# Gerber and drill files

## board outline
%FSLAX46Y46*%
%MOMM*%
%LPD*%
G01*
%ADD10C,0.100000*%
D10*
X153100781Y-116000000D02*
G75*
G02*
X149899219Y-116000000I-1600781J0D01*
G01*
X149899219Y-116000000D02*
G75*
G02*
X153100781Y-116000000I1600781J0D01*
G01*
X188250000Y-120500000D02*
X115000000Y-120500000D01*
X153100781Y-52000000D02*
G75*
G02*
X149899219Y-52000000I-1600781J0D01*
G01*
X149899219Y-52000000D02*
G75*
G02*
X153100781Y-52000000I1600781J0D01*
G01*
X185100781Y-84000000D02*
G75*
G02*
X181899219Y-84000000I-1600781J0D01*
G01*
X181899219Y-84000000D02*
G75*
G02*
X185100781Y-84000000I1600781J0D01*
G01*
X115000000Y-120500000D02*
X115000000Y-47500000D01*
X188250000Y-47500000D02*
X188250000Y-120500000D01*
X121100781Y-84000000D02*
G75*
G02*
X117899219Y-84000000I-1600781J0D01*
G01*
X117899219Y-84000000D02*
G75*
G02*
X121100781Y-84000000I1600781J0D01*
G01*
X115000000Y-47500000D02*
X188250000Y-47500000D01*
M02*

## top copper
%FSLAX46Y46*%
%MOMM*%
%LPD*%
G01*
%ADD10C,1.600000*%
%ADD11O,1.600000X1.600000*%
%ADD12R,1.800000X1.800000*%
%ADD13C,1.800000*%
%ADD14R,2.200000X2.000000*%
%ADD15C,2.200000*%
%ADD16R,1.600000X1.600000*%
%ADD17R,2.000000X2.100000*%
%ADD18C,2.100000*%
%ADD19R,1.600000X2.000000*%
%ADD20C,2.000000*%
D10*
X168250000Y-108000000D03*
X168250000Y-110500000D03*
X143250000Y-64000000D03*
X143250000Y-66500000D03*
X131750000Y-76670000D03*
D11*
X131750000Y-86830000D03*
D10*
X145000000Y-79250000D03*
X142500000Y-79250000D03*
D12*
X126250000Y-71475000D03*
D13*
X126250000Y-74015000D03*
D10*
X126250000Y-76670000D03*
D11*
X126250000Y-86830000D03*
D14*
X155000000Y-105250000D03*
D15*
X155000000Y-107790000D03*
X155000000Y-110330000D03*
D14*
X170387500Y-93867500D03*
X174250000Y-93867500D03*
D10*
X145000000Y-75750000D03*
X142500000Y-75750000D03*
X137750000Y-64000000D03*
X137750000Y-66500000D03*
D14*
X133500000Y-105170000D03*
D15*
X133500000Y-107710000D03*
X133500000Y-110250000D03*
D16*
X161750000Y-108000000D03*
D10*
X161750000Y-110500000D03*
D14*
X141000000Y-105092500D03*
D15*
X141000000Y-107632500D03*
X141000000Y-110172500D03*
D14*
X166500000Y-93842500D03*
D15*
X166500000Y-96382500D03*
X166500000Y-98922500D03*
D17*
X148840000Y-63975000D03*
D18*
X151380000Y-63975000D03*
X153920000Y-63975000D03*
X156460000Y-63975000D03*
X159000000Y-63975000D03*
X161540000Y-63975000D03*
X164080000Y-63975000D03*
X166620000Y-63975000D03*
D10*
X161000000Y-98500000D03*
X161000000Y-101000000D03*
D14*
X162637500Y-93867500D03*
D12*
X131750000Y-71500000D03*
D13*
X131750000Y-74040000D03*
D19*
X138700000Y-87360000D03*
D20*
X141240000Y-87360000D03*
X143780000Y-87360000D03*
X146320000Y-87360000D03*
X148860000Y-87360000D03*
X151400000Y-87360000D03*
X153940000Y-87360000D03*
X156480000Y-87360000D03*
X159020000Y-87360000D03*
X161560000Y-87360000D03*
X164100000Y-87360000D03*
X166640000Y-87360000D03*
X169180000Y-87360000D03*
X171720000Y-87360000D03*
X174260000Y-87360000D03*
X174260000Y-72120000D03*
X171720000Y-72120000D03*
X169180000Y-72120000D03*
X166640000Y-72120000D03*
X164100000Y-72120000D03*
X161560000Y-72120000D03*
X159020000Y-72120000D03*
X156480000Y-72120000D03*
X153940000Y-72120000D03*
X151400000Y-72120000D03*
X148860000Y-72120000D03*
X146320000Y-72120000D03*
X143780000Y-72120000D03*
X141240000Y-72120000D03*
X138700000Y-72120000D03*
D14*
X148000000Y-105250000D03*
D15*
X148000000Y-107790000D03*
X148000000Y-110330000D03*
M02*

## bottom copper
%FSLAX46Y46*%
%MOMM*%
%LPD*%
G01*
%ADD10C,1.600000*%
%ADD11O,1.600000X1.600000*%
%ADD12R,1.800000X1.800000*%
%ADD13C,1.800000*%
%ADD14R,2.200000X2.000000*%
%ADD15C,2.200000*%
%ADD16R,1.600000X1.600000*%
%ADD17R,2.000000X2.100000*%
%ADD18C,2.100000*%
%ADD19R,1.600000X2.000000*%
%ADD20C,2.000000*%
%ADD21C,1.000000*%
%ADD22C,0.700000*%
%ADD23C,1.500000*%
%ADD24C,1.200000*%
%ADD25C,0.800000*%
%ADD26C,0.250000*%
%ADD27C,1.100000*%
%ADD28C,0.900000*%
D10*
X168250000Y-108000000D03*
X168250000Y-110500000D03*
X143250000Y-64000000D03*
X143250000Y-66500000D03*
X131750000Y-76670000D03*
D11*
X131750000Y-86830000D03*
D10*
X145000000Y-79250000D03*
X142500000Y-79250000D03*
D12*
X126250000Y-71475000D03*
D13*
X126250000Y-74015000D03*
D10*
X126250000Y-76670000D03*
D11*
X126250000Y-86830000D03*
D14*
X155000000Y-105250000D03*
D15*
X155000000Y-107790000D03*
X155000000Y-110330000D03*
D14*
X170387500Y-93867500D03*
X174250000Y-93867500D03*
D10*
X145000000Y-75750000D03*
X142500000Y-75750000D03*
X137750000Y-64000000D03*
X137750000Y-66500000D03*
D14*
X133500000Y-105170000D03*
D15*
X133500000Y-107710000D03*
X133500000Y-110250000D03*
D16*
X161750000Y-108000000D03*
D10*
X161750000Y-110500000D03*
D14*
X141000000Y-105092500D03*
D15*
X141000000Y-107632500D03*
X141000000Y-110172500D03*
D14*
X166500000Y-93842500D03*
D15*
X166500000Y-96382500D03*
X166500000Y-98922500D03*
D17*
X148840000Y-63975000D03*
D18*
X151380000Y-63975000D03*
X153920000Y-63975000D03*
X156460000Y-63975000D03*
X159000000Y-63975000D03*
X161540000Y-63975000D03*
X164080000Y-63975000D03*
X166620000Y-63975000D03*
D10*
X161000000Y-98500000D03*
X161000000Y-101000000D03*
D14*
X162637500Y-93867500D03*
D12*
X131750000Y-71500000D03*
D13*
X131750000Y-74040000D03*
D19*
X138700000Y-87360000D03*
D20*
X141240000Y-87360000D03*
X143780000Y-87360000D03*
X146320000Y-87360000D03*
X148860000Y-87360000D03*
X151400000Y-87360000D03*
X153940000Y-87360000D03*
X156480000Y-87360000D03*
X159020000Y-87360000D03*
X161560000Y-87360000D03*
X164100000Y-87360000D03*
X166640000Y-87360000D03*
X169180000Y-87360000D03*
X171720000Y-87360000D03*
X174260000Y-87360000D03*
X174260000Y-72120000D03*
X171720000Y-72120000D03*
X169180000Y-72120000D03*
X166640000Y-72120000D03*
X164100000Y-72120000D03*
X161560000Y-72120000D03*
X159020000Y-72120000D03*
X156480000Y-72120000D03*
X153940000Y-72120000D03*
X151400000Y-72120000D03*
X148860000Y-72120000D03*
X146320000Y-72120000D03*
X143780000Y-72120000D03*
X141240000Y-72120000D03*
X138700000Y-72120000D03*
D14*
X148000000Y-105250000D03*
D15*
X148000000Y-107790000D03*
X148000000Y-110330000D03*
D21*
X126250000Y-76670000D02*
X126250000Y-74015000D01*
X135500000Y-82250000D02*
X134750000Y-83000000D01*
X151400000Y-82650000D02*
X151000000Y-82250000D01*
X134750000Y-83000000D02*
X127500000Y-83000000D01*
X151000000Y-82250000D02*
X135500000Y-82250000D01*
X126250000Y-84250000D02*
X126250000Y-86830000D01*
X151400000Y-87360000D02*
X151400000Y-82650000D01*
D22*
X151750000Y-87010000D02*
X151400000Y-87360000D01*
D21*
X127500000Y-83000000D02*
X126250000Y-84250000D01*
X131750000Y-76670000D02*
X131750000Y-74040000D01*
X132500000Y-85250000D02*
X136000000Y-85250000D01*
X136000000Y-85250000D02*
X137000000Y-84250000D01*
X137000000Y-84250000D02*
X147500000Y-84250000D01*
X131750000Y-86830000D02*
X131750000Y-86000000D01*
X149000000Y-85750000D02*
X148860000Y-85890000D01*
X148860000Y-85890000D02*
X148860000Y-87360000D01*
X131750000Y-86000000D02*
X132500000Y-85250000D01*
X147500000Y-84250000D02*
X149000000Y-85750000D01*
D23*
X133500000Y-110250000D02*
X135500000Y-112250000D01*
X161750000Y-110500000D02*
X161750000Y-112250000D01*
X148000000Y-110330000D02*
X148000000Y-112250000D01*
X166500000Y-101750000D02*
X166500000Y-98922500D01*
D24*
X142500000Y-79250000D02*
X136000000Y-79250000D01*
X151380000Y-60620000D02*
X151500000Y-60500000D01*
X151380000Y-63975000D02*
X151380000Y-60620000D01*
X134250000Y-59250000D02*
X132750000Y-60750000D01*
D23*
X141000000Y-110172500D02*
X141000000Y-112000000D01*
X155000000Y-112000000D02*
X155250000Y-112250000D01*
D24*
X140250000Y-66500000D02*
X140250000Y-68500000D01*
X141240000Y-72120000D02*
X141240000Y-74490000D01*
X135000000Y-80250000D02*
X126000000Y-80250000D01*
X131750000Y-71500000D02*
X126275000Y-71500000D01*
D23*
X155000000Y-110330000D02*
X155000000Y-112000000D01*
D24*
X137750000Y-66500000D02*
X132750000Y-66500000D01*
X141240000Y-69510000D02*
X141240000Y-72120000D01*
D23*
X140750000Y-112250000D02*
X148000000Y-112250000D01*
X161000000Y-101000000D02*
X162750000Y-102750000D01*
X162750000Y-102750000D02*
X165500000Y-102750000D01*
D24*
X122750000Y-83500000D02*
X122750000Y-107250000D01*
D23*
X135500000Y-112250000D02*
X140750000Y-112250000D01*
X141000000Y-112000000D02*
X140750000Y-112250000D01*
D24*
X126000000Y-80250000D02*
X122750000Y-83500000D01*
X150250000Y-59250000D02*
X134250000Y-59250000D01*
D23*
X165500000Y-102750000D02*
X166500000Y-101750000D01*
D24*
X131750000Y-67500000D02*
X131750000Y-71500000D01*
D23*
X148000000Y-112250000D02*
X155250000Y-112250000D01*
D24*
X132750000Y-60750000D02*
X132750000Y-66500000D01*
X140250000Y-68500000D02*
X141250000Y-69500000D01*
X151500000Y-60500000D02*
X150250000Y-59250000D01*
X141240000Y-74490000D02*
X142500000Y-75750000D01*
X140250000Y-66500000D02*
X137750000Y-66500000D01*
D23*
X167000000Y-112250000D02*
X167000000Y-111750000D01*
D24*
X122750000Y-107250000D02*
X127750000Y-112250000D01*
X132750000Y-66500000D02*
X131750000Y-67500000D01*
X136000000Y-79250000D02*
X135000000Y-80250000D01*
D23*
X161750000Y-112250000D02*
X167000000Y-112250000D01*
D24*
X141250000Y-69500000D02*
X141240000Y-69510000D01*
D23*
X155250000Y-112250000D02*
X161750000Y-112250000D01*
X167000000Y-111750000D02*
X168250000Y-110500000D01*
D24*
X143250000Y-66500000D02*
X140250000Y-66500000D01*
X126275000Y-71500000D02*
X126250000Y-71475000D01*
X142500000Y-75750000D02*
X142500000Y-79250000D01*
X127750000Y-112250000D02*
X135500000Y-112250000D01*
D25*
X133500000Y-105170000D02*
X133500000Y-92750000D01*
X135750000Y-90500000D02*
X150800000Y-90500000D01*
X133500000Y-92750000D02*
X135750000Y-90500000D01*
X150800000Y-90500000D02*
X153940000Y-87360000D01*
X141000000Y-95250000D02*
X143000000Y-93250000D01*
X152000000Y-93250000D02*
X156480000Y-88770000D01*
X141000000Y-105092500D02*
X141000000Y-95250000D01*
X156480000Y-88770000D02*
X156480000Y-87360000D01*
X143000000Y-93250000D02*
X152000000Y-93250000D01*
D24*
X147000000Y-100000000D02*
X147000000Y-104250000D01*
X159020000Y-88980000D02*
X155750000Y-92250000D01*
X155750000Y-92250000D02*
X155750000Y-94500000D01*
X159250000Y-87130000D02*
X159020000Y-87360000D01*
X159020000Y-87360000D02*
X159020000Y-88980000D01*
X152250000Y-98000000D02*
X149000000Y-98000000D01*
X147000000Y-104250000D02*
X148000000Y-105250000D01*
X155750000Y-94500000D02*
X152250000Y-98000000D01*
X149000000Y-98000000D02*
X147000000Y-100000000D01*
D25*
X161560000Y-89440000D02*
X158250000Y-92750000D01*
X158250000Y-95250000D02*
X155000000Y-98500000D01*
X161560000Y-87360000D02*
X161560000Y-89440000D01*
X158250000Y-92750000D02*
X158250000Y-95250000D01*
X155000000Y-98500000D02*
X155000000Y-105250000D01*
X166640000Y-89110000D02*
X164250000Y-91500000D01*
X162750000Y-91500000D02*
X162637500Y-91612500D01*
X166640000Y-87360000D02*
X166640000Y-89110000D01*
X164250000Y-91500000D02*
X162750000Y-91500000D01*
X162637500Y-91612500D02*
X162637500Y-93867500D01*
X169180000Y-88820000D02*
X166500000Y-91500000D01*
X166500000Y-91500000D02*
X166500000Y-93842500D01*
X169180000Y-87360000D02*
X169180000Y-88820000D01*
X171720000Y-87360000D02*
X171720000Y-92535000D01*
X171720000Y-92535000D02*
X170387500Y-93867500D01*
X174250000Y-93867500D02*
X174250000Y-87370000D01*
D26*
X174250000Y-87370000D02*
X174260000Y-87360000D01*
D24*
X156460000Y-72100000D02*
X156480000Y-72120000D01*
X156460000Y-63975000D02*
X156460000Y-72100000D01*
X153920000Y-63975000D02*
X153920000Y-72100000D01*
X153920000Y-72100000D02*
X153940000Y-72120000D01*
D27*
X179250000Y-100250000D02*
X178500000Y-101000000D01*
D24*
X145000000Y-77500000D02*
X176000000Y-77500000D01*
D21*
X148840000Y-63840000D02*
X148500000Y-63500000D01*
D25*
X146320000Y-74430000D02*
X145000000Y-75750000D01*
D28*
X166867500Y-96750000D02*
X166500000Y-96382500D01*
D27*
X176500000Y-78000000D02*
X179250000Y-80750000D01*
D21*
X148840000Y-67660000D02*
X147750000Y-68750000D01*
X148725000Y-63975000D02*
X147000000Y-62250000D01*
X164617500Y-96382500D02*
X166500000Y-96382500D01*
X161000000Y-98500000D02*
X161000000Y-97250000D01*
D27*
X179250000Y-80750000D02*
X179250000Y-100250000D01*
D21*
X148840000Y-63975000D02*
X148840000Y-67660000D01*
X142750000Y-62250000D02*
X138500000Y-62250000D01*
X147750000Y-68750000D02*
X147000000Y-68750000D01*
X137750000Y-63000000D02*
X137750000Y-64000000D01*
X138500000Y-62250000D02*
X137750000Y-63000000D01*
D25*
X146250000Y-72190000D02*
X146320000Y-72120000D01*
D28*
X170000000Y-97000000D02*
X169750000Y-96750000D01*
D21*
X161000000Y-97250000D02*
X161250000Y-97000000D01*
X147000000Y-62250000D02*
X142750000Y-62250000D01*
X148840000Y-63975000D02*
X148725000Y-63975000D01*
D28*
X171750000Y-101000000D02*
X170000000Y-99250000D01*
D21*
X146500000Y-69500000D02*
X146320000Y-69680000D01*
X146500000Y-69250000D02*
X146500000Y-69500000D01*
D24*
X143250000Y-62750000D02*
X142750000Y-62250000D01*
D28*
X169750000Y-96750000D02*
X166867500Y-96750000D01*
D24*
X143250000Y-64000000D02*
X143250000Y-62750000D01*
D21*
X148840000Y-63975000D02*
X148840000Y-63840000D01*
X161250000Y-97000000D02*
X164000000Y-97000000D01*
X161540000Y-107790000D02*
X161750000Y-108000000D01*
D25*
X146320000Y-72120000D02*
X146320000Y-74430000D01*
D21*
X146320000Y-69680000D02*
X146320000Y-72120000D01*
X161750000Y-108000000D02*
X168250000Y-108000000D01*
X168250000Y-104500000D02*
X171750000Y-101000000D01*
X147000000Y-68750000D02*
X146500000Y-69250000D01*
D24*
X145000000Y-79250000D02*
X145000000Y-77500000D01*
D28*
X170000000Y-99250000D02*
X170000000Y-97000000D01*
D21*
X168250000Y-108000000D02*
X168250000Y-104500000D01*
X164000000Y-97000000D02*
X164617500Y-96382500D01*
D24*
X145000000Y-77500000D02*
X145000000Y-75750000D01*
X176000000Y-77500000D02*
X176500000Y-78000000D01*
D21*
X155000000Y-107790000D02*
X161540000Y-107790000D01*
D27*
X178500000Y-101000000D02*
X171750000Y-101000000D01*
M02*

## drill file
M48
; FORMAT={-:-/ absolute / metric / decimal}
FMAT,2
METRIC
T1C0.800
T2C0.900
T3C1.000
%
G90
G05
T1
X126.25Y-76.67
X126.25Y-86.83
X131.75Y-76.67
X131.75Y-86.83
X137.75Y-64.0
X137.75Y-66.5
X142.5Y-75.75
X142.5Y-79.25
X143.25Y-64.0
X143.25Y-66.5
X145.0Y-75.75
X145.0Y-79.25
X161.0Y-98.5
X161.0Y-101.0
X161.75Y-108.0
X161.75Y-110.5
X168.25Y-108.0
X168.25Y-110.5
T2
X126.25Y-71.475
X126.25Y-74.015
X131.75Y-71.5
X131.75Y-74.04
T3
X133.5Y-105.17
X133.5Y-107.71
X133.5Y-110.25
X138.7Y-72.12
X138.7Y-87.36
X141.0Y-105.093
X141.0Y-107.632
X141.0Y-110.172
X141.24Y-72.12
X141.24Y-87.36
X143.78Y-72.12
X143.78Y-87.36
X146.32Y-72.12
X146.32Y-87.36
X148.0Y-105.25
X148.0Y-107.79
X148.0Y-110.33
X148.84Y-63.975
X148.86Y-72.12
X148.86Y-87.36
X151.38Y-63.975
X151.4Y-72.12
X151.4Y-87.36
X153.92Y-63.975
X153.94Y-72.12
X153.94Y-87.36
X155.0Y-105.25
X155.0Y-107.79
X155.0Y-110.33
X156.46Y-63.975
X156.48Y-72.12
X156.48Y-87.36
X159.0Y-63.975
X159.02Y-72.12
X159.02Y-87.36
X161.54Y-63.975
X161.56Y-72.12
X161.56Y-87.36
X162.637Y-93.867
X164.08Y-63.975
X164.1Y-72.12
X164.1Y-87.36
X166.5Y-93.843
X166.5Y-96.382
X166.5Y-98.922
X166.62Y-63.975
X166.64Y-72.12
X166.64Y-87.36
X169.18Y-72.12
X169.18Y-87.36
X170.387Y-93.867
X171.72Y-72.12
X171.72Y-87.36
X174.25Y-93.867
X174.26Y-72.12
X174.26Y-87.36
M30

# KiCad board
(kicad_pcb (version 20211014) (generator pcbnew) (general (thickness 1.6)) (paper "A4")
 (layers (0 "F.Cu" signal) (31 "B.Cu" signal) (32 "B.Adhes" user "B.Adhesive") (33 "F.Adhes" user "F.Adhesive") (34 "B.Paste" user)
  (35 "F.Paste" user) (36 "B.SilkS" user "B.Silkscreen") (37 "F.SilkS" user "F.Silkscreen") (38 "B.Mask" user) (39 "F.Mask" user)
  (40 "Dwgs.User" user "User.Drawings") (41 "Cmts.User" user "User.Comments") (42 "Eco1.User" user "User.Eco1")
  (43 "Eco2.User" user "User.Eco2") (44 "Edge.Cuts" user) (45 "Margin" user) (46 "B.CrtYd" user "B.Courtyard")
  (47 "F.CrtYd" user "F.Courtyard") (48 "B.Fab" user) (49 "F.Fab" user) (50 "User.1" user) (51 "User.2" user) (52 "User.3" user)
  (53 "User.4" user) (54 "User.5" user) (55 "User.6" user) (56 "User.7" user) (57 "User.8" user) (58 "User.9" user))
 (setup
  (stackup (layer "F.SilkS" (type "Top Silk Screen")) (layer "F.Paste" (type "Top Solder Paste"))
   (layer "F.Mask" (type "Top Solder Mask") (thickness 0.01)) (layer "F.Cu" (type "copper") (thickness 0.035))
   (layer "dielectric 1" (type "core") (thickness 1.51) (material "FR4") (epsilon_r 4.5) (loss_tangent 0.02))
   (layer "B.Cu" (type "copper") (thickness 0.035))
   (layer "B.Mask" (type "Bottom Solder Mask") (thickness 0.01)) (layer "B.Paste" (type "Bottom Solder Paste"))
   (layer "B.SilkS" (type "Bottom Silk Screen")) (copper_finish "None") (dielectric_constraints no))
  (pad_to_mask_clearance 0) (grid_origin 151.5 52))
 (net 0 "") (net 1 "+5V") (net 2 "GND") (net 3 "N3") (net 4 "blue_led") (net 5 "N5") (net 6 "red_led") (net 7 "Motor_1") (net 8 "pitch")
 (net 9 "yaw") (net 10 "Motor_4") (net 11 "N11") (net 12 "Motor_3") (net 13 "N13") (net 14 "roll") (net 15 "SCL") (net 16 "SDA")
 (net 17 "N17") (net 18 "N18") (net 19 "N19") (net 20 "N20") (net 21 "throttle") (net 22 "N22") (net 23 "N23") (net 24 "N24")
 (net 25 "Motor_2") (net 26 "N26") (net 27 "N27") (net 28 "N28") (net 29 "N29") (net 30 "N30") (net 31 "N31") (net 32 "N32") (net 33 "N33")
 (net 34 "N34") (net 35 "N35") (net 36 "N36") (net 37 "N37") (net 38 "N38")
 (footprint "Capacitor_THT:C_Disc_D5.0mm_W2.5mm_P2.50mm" (layer "F.Cu") (at 168.25 108 -90)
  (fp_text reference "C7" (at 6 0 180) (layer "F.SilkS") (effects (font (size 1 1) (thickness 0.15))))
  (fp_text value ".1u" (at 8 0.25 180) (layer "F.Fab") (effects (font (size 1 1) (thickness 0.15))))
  (pad "1" thru_hole circle (at 0 0 270) (size 1.6 1.6) (drill 0.8) (layers *.Cu *.Mask) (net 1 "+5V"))
  (pad "2" thru_hole circle (at 2.5 0 270) (size 1.6 1.6) (drill 0.8) (layers *.Cu *.Mask) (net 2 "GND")))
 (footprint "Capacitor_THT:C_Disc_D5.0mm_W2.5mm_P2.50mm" (layer "F.Cu") (at 143.25 64 -90)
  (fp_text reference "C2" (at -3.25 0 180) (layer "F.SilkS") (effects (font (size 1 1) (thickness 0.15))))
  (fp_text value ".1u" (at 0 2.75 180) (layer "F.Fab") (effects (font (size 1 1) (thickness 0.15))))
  (pad "1" thru_hole circle (at 0 0 270) (size 1.6 1.6) (drill 0.8) (layers *.Cu *.Mask) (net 1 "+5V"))
  (pad "2" thru_hole circle (at 2.5 0 270) (size 1.6 1.6) (drill 0.8) (layers *.Cu *.Mask) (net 2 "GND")))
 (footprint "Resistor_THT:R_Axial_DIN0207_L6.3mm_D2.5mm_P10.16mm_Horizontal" (layer "F.Cu") (at 131.75 76.67 -90)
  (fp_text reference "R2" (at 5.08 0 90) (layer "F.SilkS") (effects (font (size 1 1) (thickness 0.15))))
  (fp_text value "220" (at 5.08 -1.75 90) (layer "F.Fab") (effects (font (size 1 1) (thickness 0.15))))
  (pad "1" thru_hole circle (at 0 0 270) (size 1.6 1.6) (drill 0.8) (layers *.Cu *.Mask) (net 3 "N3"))
  (pad "2" thru_hole oval (at 10.16 0 270) (size 1.6 1.6) (drill 0.8) (layers *.Cu *.Mask) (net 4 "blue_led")))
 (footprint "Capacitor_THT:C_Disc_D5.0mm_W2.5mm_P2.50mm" (layer "F.Cu") (at 145 79.25 180)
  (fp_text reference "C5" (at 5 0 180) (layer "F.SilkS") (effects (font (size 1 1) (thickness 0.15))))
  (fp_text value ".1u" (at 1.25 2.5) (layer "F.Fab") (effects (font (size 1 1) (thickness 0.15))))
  (pad "1" thru_hole circle (at 0 0 180) (size 1.6 1.6) (drill 0.8) (layers *.Cu *.Mask) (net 1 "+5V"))
  (pad "2" thru_hole circle (at 2.5 0 180) (size 1.6 1.6) (drill 0.8) (layers *.Cu *.Mask) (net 2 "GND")))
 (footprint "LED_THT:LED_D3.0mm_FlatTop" (layer "F.Cu") (at 126.25 71.475 -90)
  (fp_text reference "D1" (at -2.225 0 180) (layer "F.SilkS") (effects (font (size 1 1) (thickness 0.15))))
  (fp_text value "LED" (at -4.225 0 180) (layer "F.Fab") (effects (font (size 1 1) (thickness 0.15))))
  (pad "1" thru_hole rect (at 0 0 270) (size 1.8 1.8) (drill 0.9) (layers *.Cu *.Mask) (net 2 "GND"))
  (pad "2" thru_hole circle (at 2.54 0 270) (size 1.8 1.8) (drill 0.9) (layers *.Cu *.Mask) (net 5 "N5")))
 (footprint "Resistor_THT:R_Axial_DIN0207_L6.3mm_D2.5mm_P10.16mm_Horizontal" (layer "F.Cu") (at 126.25 76.67 -90)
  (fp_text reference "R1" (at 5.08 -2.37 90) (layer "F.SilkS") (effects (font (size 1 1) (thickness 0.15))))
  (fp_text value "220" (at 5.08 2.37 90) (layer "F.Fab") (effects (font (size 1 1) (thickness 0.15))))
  (pad "1" thru_hole circle (at 0 0 270) (size 1.6 1.6) (drill 0.8) (layers *.Cu *.Mask) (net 5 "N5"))
  (pad "2" thru_hole oval (at 10.16 0 270) (size 1.6 1.6) (drill 0.8) (layers *.Cu *.Mask) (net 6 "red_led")))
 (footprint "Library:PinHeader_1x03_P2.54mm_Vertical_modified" (layer "F.Cu") (at 156.33 114.14)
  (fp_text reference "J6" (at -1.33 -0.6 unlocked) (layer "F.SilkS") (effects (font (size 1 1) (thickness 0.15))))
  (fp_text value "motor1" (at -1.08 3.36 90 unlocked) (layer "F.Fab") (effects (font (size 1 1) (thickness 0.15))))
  (pad "1" thru_hole rect (at -1.33 -8.89) (size 2.2 2) (drill 1) (layers *.Cu *.Mask) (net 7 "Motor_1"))
  (pad "2" thru_hole circle (at -1.33 -6.35) (size 2.2 2.2) (drill 1) (layers *.Cu *.Mask) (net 1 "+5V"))
  (pad "3" thru_hole circle (at -1.33 -3.81) (size 2.2 2.2) (drill 1) (layers *.Cu *.Mask) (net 2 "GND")))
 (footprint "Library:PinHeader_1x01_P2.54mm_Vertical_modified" (layer "F.Cu") (at 172.1875 98.2075)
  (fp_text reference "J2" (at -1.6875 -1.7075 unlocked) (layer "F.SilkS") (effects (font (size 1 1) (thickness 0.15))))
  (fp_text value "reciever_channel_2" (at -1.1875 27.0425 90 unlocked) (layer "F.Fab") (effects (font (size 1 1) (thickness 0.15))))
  (pad "1" thru_hole rect (at -1.8 -4.34) (size 2.2 2) (drill 1) (layers *.Cu *.Mask) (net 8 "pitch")))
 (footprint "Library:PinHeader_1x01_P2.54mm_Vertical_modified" (layer "F.Cu") (at 176.05 98.2075)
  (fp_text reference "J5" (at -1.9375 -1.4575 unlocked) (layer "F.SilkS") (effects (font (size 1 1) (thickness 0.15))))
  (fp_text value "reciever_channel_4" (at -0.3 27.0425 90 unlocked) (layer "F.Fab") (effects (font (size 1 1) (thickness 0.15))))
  (pad "1" thru_hole rect (at -1.8 -4.34) (size 2.2 2) (drill 1) (layers *.Cu *.Mask) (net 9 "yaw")))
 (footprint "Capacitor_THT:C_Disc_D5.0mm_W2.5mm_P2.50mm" (layer "F.Cu") (at 145 75.75 180)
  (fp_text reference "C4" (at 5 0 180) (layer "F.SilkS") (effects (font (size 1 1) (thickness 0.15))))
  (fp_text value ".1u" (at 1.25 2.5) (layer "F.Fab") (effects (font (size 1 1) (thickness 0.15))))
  (pad "1" thru_hole circle (at 0 0 180) (size 1.6 1.6) (drill 0.8) (layers *.Cu *.Mask) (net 1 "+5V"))
  (pad "2" thru_hole circle (at 2.5 0 180) (size 1.6 1.6) (drill 0.8) (layers *.Cu *.Mask) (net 2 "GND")))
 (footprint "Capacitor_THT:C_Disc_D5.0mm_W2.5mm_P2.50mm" (layer "F.Cu") (at 137.75 64 -90)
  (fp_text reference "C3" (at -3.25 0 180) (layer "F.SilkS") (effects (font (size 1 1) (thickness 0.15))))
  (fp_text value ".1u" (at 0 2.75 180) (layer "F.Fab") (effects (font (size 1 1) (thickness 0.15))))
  (pad "1" thru_hole circle (at 0 0 270) (size 1.6 1.6) (drill 0.8) (layers *.Cu *.Mask) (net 1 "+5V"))
  (pad "2" thru_hole circle (at 2.5 0 270) (size 1.6 1.6) (drill 0.8) (layers *.Cu *.Mask) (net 2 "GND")))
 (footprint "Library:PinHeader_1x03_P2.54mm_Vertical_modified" (layer "F.Cu") (at 134.83 114.06)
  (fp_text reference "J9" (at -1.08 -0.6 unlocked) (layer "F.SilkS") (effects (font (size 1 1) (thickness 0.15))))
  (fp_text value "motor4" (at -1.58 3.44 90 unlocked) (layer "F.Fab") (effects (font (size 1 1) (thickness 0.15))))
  (pad "1" thru_hole rect (at -1.33 -8.89) (size 2.2 2) (drill 1) (layers *.Cu *.Mask) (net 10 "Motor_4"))
  (pad "2" thru_hole circle (at -1.33 -6.35) (size 2.2 2.2) (drill 1) (layers *.Cu *.Mask) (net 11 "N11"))
  (pad "3" thru_hole circle (at -1.33 -3.81) (size 2.2 2.2) (drill 1) (layers *.Cu *.Mask) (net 2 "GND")))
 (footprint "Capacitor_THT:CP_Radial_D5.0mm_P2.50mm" (layer "F.Cu") (at 161.75 108 -90)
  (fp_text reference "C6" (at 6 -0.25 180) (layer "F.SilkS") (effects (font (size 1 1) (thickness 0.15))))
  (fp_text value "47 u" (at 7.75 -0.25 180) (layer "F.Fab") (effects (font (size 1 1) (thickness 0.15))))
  (pad "1" thru_hole rect (at 0 0 270) (size 1.6 1.6) (drill 0.8) (layers *.Cu *.Mask) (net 1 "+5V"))
  (pad "2" thru_hole circle (at 2.5 0 270) (size 1.6 1.6) (drill 0.8) (layers *.Cu *.Mask) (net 2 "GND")))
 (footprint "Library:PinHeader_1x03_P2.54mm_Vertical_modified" (layer "F.Cu") (at 142.33 113.9825)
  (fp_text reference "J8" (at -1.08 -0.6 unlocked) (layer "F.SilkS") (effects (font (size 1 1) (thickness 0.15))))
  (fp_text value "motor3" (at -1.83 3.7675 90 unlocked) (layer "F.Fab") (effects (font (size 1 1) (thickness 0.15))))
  (pad "1" thru_hole rect (at -1.33 -8.89) (size 2.2 2) (drill 1) (layers *.Cu *.Mask) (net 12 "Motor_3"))
  (pad "2" thru_hole circle (at -1.33 -6.35) (size 2.2 2.2) (drill 1) (layers *.Cu *.Mask) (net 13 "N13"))
  (pad "3" thru_hole circle (at -1.33 -3.81) (size 2.2 2.2) (drill 1) (layers *.Cu *.Mask) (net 2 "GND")))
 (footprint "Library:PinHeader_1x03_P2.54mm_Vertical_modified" (layer "F.Cu") (at 167.83 102.7325)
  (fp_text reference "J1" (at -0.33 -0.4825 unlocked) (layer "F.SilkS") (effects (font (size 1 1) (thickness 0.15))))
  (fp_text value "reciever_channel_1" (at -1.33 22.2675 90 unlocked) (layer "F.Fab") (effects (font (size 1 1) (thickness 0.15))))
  (pad "1" thru_hole rect (at -1.33 -8.89) (size 2.2 2) (drill 1) (layers *.Cu *.Mask) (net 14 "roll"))
  (pad "2" thru_hole circle (at -1.33 -6.35) (size 2.2 2.2) (drill 1) (layers *.Cu *.Mask) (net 1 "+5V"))
  (pad "3" thru_hole circle (at -1.33 -3.81) (size 2.2 2.2) (drill 1) (layers *.Cu *.Mask) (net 2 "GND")))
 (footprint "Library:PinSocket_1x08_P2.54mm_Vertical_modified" (layer "F.Cu") (at 170.49 65.185 90)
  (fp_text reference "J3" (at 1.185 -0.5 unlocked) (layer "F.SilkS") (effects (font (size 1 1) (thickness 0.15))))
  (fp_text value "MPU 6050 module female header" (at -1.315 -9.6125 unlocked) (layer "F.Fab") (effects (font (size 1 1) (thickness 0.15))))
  (pad "1" thru_hole rect (at 1.21 -21.65 90) (size 2.1 2) (drill 1) (layers *.Cu *.Mask) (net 1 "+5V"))
  (pad "2" thru_hole circle (at 1.21 -19.11 90) (size 2.1 2.1) (drill 1) (layers *.Cu *.Mask) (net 2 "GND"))
  (pad "3" thru_hole circle (at 1.21 -16.57 90) (size 2.1 2.1) (drill 1) (layers *.Cu *.Mask) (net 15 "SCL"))
  (pad "4" thru_hole circle (at 1.21 -14.03 90) (size 2.1 2.1) (drill 1) (layers *.Cu *.Mask) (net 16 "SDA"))
  (pad "5" thru_hole circle (at 1.21 -11.49 90) (size 2.1 2.1) (drill 1) (layers *.Cu *.Mask) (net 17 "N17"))
  (pad "6" thru_hole circle (at 1.21 -8.95 90) (size 2.1 2.1) (drill 1) (layers *.Cu *.Mask) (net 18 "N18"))
  (pad "7" thru_hole circle (at 1.21 -6.41 90) (size 2.1 2.1) (drill 1) (layers *.Cu *.Mask) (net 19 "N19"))
  (pad "8" thru_hole circle (at 1.21 -3.87 90) (size 2.1 2.1) (drill 1) (layers *.Cu *.Mask) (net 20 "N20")))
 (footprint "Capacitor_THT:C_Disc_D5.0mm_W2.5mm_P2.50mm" (layer "F.Cu") (at 161 98.5 -90)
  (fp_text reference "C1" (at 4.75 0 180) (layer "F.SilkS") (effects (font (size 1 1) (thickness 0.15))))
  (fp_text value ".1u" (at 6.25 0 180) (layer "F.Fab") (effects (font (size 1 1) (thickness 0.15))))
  (pad "1" thru_hole circle (at 0 0 270) (size 1.6 1.6) (drill 0.8) (layers *.Cu *.Mask) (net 1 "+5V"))
  (pad "2" thru_hole circle (at 2.5 0 270) (size 1.6 1.6) (drill 0.8) (layers *.Cu *.Mask) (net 2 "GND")))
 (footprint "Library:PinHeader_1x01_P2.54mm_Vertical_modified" (layer "F.Cu") (at 164.4375 98.2075)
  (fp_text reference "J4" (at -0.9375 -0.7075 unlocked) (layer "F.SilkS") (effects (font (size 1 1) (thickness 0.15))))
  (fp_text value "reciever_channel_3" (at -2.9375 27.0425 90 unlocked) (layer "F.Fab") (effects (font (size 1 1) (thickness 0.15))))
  (pad "1" thru_hole rect (at -1.8 -4.34) (size 2.2 2) (drill 1) (layers *.Cu *.Mask) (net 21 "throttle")))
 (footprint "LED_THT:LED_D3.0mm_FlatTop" (layer "F.Cu") (at 131.75 71.5 -90)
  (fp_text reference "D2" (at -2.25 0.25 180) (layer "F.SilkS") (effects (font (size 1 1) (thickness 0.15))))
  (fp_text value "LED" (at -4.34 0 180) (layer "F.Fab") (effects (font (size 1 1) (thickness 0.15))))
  (pad "1" thru_hole rect (at 0 0 270) (size 1.8 1.8) (drill 0.9) (layers *.Cu *.Mask) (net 2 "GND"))
  (pad "2" thru_hole circle (at 2.54 0 270) (size 1.8 1.8) (drill 0.9) (layers *.Cu *.Mask) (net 3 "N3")))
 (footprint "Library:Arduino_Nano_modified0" (layer "F.Cu") (at 138.7 87.36 90)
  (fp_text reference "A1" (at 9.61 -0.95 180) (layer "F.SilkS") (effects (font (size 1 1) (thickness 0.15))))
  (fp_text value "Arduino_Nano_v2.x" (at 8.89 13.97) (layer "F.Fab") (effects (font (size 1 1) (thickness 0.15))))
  (pad "1" thru_hole rect (at 0 0 90) (size 2 1.6) (drill 1) (layers *.Cu *.Mask) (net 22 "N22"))
  (pad "2" thru_hole circle (at 0 2.54 90) (size 2 2) (drill 1) (layers *.Cu *.Mask) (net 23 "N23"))
  (pad "3" thru_hole circle (at 0 5.08 90) (size 2 2) (drill 1) (layers *.Cu *.Mask) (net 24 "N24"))
  (pad "4" thru_hole circle (at 0 7.62 90) (size 2 2) (drill 1) (layers *.Cu *.Mask) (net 2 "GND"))
  (pad "5" thru_hole circle (at 0 10.16 90) (size 2 2) (drill 1) (layers *.Cu *.Mask) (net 4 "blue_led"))
  (pad "6" thru_hole circle (at 0 12.7 90) (size 2 2) (drill 1) (layers *.Cu *.Mask) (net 6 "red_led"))
  (pad "7" thru_hole circle (at 0 15.24 90) (size 2 2) (drill 1) (layers *.Cu *.Mask) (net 10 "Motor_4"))
  (pad "8" thru_hole circle (at 0 17.78 90) (size 2 2) (drill 1) (layers *.Cu *.Mask) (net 12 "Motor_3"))
  (pad "9" thru_hole circle (at 0 20.32 90) (size 2 2) (drill 1) (layers *.Cu *.Mask) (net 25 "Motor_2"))
  (pad "10" thru_hole circle (at 0 22.86 90) (size 2 2) (drill 1) (layers *.Cu *.Mask) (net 7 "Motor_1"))
  (pad "11" thru_hole circle (at 0 25.4 90) (size 2 2) (drill 1) (layers *.Cu *.Mask) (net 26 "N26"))
  (pad "12" thru_hole circle (at 0 27.94 90) (size 2 2) (drill 1) (layers *.Cu *.Mask) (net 21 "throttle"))
  (pad "13" thru_hole circle (at 0 30.48 90) (size 2 2) (drill 1) (layers *.Cu *.Mask) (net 14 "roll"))
  (pad "14" thru_hole circle (at 0 33.02 90) (size 2 2) (drill 1) (layers *.Cu *.Mask) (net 8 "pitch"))
  (pad "15" thru_hole circle (at 0 35.56 90) (size 2 2) (drill 1) (layers *.Cu *.Mask) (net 9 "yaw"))
  (pad "16" thru_hole circle (at 15.24 35.56 90) (size 2 2) (drill 1) (layers *.Cu *.Mask) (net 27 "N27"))
  (pad "17" thru_hole circle (at 15.24 33.02 90) (size 2 2) (drill 1) (layers *.Cu *.Mask) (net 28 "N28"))
  (pad "18" thru_hole circle (at 15.24 30.48 90) (size 2 2) (drill 1) (layers *.Cu *.Mask) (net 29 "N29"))
  (pad "19" thru_hole circle (at 15.24 27.94 90) (size 2 2) (drill 1) (layers *.Cu *.Mask) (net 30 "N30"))
  (pad "20" thru_hole circle (at 15.24 25.4 90) (size 2 2) (drill 1) (layers *.Cu *.Mask) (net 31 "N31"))
  (pad "21" thru_hole circle (at 15.24 22.86 90) (size 2 2) (drill 1) (layers *.Cu *.Mask) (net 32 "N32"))
  (pad "22" thru_hole circle (at 15.24 20.32 90) (size 2 2) (drill 1) (layers *.Cu *.Mask) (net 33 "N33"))
  (pad "23" thru_hole circle (at 15.24 17.78 90) (size 2 2) (drill 1) (layers *.Cu *.Mask) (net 16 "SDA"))
  (pad "24" thru_hole circle (at 15.24 15.24 90) (size 2 2) (drill 1) (layers *.Cu *.Mask) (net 15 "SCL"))
  (pad "25" thru_hole circle (at 15.24 12.7 90) (size 2 2) (drill 1) (layers *.Cu *.Mask) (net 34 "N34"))
  (pad "26" thru_hole circle (at 15.24 10.16 90) (size 2 2) (drill 1) (layers *.Cu *.Mask) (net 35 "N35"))
  (pad "27" thru_hole circle (at 15.24 7.62 90) (size 2 2) (drill 1) (layers *.Cu *.Mask) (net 1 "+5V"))
  (pad "28" thru_hole circle (at 15.24 5.08 90) (size 2 2) (drill 1) (layers *.Cu *.Mask) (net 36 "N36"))
  (pad "29" thru_hole circle (at 15.24 2.54 90) (size 2 2) (drill 1) (layers *.Cu *.Mask) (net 2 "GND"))
  (pad "30" thru_hole circle (at 15.24 0 90) (size 2 2) (drill 1) (layers *.Cu *.Mask) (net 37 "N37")))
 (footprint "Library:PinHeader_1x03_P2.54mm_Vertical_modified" (layer "F.Cu") (at 149.33 114.14)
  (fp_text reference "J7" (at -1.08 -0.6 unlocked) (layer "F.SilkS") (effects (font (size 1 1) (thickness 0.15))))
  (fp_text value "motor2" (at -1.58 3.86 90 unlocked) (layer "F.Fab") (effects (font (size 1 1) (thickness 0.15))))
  (pad "1" thru_hole rect (at -1.33 -8.89) (size 2.2 2) (drill 1) (layers *.Cu *.Mask) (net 25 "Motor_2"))
  (pad "2" thru_hole circle (at -1.33 -6.35) (size 2.2 2.2) (drill 1) (layers *.Cu *.Mask) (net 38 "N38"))
  (pad "3" thru_hole circle (at -1.33 -3.81) (size 2.2 2.2) (drill 1) (layers *.Cu *.Mask) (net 2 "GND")))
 (gr_circle (center 151.5 116) (end 152.75 115) (layer "Edge.Cuts") (width 0.1) (fill none))
 (gr_line (start 188.25 120.5) (end 115 120.5) (layer "Edge.Cuts") (width 0.1))
 (gr_circle (center 151.5 52) (end 152.75 51) (layer "Edge.Cuts") (width 0.1) (fill none))
 (gr_circle (center 183.5 84) (end 184.5 82.75) (layer "Edge.Cuts") (width 0.1) (fill none))
 (gr_line (start 115 120.5) (end 115 47.5) (layer "Edge.Cuts") (width 0.1))
 (gr_line (start 188.25 47.5) (end 188.25 120.5) (layer "Edge.Cuts") (width 0.1))
 (gr_circle (center 119.5 84) (end 120.5 82.75) (layer "Edge.Cuts") (width 0.1) (fill none))
 (gr_line (start 115 47.5) (end 188.25 47.5) (layer "Edge.Cuts") (width 0.1))
 (segment (start 126.25 76.67) (end 126.25 74.015) (width 1) (layer "B.Cu") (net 5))
 (segment (start 135.5 82.25) (end 134.75 83) (width 1) (layer "B.Cu") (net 6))
 (segment (start 151.4 82.65) (end 151 82.25) (width 1) (layer "B.Cu") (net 6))
 (segment (start 134.75 83) (end 127.5 83) (width 1) (layer "B.Cu") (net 6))
 (segment (start 151 82.25) (end 135.5 82.25) (width 1) (layer "B.Cu") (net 6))
 (segment (start 126.25 84.25) (end 126.25 86.83) (width 1) (layer "B.Cu") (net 6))
 (segment (start 151.4 87.36) (end 151.4 82.65) (width 1) (layer "B.Cu") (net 6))
 (segment (start 151.75 87.01) (end 151.4 87.36) (width 0.7) (layer "B.Cu") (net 6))
 (segment (start 127.5 83) (end 126.25 84.25) (width 1) (layer "B.Cu") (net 6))
 (segment (start 131.75 76.67) (end 131.75 74.04) (width 1) (layer "B.Cu") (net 3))
 (segment (start 132.5 85.25) (end 136 85.25) (width 1) (layer "B.Cu") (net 4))
 (segment (start 136 85.25) (end 137 84.25) (width 1) (layer "B.Cu") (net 4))
 (segment (start 137 84.25) (end 147.5 84.25) (width 1) (layer "B.Cu") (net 4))
 (segment (start 131.75 86.83) (end 131.75 86) (width 1) (layer "B.Cu") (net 4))
 (segment (start 149 85.75) (end 148.86 85.89) (width 1) (layer "B.Cu") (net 4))
 (segment (start 148.86 85.89) (end 148.86 87.36) (width 1) (layer "B.Cu") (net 4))
 (segment (start 131.75 86) (end 132.5 85.25) (width 1) (layer "B.Cu") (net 4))
 (segment (start 147.5 84.25) (end 149 85.75) (width 1) (layer "B.Cu") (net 4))
 (segment (start 133.5 110.25) (end 135.5 112.25) (width 1.5) (layer "B.Cu") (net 2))
 (segment (start 161.75 110.5) (end 161.75 112.25) (width 1.5) (layer "B.Cu") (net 2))
 (segment (start 148 110.33) (end 148 112.25) (width 1.5) (layer "B.Cu") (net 2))
 (segment (start 166.5 101.75) (end 166.5 98.9225) (width 1.5) (layer "B.Cu") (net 2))
 (segment (start 142.5 79.25) (end 136 79.25) (width 1.2) (layer "B.Cu") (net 2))
 (segment (start 151.38 60.62) (end 151.5 60.5) (width 1.2) (layer "B.Cu") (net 2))
 (segment (start 151.38 63.975) (end 151.38 60.62) (width 1.2) (layer "B.Cu") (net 2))
 (segment (start 134.25 59.25) (end 132.75 60.75) (width 1.2) (layer "B.Cu") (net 2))
 (segment (start 141 110.1725) (end 141 112) (width 1.5) (layer "B.Cu") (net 2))
 (segment (start 155 112) (end 155.25 112.25) (width 1.5) (layer "B.Cu") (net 2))
 (segment (start 140.25 66.5) (end 140.25 68.5) (width 1.2) (layer "B.Cu") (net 2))
 (segment (start 141.24 72.12) (end 141.24 74.49) (width 1.2) (layer "B.Cu") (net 2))
 (segment (start 135 80.25) (end 126 80.25) (width 1.2) (layer "B.Cu") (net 2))
 (segment (start 131.75 71.5) (end 126.275 71.5) (width 1.2) (layer "B.Cu") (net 2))
 (segment (start 155 110.33) (end 155 112) (width 1.5) (layer "B.Cu") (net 2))
 (segment (start 137.75 66.5) (end 132.75 66.5) (width 1.2) (layer "B.Cu") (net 2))
 (segment (start 141.24 69.51) (end 141.24 72.12) (width 1.2) (layer "B.Cu") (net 2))
 (segment (start 140.75 112.25) (end 148 112.25) (width 1.5) (layer "B.Cu") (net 2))
 (segment (start 161 101) (end 162.75 102.75) (width 1.5) (layer "B.Cu") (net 2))
 (segment (start 162.75 102.75) (end 165.5 102.75) (width 1.5) (layer "B.Cu") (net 2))
 (segment (start 122.75 83.5) (end 122.75 107.25) (width 1.2) (layer "B.Cu") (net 2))
 (segment (start 135.5 112.25) (end 140.75 112.25) (width 1.5) (layer "B.Cu") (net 2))
 (segment (start 141 112) (end 140.75 112.25) (width 1.5) (layer "B.Cu") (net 2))
 (segment (start 126 80.25) (end 122.75 83.5) (width 1.2) (layer "B.Cu") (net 2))
 (segment (start 150.25 59.25) (end 134.25 59.25) (width 1.2) (layer "B.Cu") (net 2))
 (segment (start 165.5 102.75) (end 166.5 101.75) (width 1.5) (layer "B.Cu") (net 2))
 (segment (start 131.75 67.5) (end 131.75 71.5) (width 1.2) (layer "B.Cu") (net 2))
 (segment (start 148 112.25) (end 155.25 112.25) (width 1.5) (layer "B.Cu") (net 2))
 (segment (start 132.75 60.75) (end 132.75 66.5) (width 1.2) (layer "B.Cu") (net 2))
 (segment (start 140.25 68.5) (end 141.25 69.5) (width 1.2) (layer "B.Cu") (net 2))
 (segment (start 151.5 60.5) (end 150.25 59.25) (width 1.2) (layer "B.Cu") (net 2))
 (segment (start 141.24 74.49) (end 142.5 75.75) (width 1.2) (layer "B.Cu") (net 2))
 (segment (start 140.25 66.5) (end 137.75 66.5) (width 1.2) (layer "B.Cu") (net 2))
 (segment (start 167 112.25) (end 167 111.75) (width 1.5) (layer "B.Cu") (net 2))
 (segment (start 122.75 107.25) (end 127.75 112.25) (width 1.2) (layer "B.Cu") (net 2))
 (segment (start 132.75 66.5) (end 131.75 67.5) (width 1.2) (layer "B.Cu") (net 2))
 (segment (start 136 79.25) (end 135 80.25) (width 1.2) (layer "B.Cu") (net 2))
 (segment (start 161.75 112.25) (end 167 112.25) (width 1.5) (layer "B.Cu") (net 2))
 (segment (start 141.25 69.5) (end 141.24 69.51) (width 1.2) (layer "B.Cu") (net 2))
 (segment (start 155.25 112.25) (end 161.75 112.25) (width 1.5) (layer "B.Cu") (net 2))
 (segment (start 167 111.75) (end 168.25 110.5) (width 1.5) (layer "B.Cu") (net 2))
 (segment (start 143.25 66.5) (end 140.25 66.5) (width 1.2) (layer "B.Cu") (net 2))
 (segment (start 126.275 71.5) (end 126.25 71.475) (width 1.2) (layer "B.Cu") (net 2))
 (segment (start 142.5 75.75) (end 142.5 79.25) (width 1.2) (layer "B.Cu") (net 2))
 (segment (start 127.75 112.25) (end 135.5 112.25) (width 1.2) (layer "B.Cu") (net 2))
 (segment (start 133.5 105.17) (end 133.5 92.75) (width 0.8) (layer "B.Cu") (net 10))
 (segment (start 135.75 90.5) (end 150.8 90.5) (width 0.8) (layer "B.Cu") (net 10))
 (segment (start 133.5 92.75) (end 135.75 90.5) (width 0.8) (layer "B.Cu") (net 10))
 (segment (start 150.8 90.5) (end 153.94 87.36) (width 0.8) (layer "B.Cu") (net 10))
 (segment (start 141 95.25) (end 143 93.25) (width 0.8) (layer "B.Cu") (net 12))
 (segment (start 152 93.25) (end 156.48 88.77) (width 0.8) (layer "B.Cu") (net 12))
 (segment (start 141 105.0925) (end 141 95.25) (width 0.8) (layer "B.Cu") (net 12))
 (segment (start 156.48 88.77) (end 156.48 87.36) (width 0.8) (layer "B.Cu") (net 12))
 (segment (start 143 93.25) (end 152 93.25) (width 0.8) (layer "B.Cu") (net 12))
 (segment (start 147 100) (end 147 104.25) (width 1.2) (layer "B.Cu") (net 25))
 (segment (start 159.02 88.98) (end 155.75 92.25) (width 1.2) (layer "B.Cu") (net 25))
 (segment (start 155.75 92.25) (end 155.75 94.5) (width 1.2) (layer "B.Cu") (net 25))
 (segment (start 159.25 87.13) (end 159.02 87.36) (width 1.2) (layer "B.Cu") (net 25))
 (segment (start 159.02 87.36) (end 159.02 88.98) (width 1.2) (layer "B.Cu") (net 25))
 (segment (start 152.25 98) (end 149 98) (width 1.2) (layer "B.Cu") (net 25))
 (segment (start 147 104.25) (end 148 105.25) (width 1.2) (layer "B.Cu") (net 25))
 (segment (start 155.75 94.5) (end 152.25 98) (width 1.2) (layer "B.Cu") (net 25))
 (segment (start 149 98) (end 147 100) (width 1.2) (layer "B.Cu") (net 25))
 (segment (start 161.56 89.44) (end 158.25 92.75) (width 0.8) (layer "B.Cu") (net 7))
 (segment (start 158.25 95.25) (end 155 98.5) (width 0.8) (layer "B.Cu") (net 7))
 (segment (start 161.56 87.36) (end 161.56 89.44) (width 0.8) (layer "B.Cu") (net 7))
 (segment (start 158.25 92.75) (end 158.25 95.25) (width 0.8) (layer "B.Cu") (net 7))
 (segment (start 155 98.5) (end 155 105.25) (width 0.8) (layer "B.Cu") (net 7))
 (segment (start 166.64 89.11) (end 164.25 91.5) (width 0.8) (layer "B.Cu") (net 21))
 (segment (start 162.75 91.5) (end 162.6375 91.6125) (width 0.8) (layer "B.Cu") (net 21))
 (segment (start 166.64 87.36) (end 166.64 89.11) (width 0.8) (layer "B.Cu") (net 21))
 (segment (start 164.25 91.5) (end 162.75 91.5) (width 0.8) (layer "B.Cu") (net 21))
 (segment (start 162.6375 91.6125) (end 162.6375 93.8675) (width 0.8) (layer "B.Cu") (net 21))
 (segment (start 169.18 88.82) (end 166.5 91.5) (width 0.8) (layer "B.Cu") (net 14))
 (segment (start 166.5 91.5) (end 166.5 93.8425) (width 0.8) (layer "B.Cu") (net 14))
 (segment (start 169.18 87.36) (end 169.18 88.82) (width 0.8) (layer "B.Cu") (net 14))
 (segment (start 171.72 87.36) (end 171.72 92.535) (width 0.8) (layer "B.Cu") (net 8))
 (segment (start 171.72 92.535) (end 170.3875 93.8675) (width 0.8) (layer "B.Cu") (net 8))
 (segment (start 174.25 93.8675) (end 174.25 87.37) (width 0.8) (layer "B.Cu") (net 9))
 (segment (start 174.25 87.37) (end 174.26 87.36) (width 0.25) (layer "B.Cu") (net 9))
 (segment (start 156.46 72.1) (end 156.48 72.12) (width 1.2) (layer "B.Cu") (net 16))
 (segment (start 156.46 63.975) (end 156.46 72.1) (width 1.2) (layer "B.Cu") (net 16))
 (segment (start 153.92 63.975) (end 153.92 72.1) (width 1.2) (layer "B.Cu") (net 15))
 (segment (start 153.92 72.1) (end 153.94 72.12) (width 1.2) (layer "B.Cu") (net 15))
 (segment (start 179.25 100.25) (end 178.5 101) (width 1.1) (layer "B.Cu") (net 1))
 (segment (start 145 77.5) (end 176 77.5) (width 1.2) (layer "B.Cu") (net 1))
 (segment (start 148.84 63.84) (end 148.5 63.5) (width 1) (layer "B.Cu") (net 1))
 (segment (start 146.32 74.43) (end 145 75.75) (width 0.8) (layer "B.Cu") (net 1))
 (segment (start 166.8675 96.75) (end 166.5 96.3825) (width 0.9) (layer "B.Cu") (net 1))
 (segment (start 176.5 78) (end 179.25 80.75) (width 1.1) (layer "B.Cu") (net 1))
 (segment (start 148.84 67.66) (end 147.75 68.75) (width 1) (layer "B.Cu") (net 1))
 (segment (start 148.725 63.975) (end 147 62.25) (width 1) (layer "B.Cu") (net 1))
 (segment (start 164.6175 96.3825) (end 166.5 96.3825) (width 1) (layer "B.Cu") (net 1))
 (segment (start 161 98.5) (end 161 97.25) (width 1) (layer "B.Cu") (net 1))
 (segment (start 179.25 80.75) (end 179.25 100.25) (width 1.1) (layer "B.Cu") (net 1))
 (segment (start 148.84 63.975) (end 148.84 67.66) (width 1) (layer "B.Cu") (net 1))
 (segment (start 142.75 62.25) (end 138.5 62.25) (width 1) (layer "B.Cu") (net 1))
 (segment (start 147.75 68.75) (end 147 68.75) (width 1) (layer "B.Cu") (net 1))
 (segment (start 137.75 63) (end 137.75 64) (width 1) (layer "B.Cu") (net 1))
 (segment (start 138.5 62.25) (end 137.75 63) (width 1) (layer "B.Cu") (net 1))
 (segment (start 146.25 72.19) (end 146.32 72.12) (width 0.8) (layer "B.Cu") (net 1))
 (segment (start 170 97) (end 169.75 96.75) (width 0.9) (layer "B.Cu") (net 1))
 (segment (start 161 97.25) (end 161.25 97) (width 1) (layer "B.Cu") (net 1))
 (segment (start 147 62.25) (end 142.75 62.25) (width 1) (layer "B.Cu") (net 1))
 (segment (start 148.84 63.975) (end 148.725 63.975) (width 1) (layer "B.Cu") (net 1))
 (segment (start 171.75 101) (end 170 99.25) (width 0.9) (layer "B.Cu") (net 1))
 (segment (start 146.5 69.5) (end 146.32 69.68) (width 1) (layer "B.Cu") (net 1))
 (segment (start 146.5 69.25) (end 146.5 69.5) (width 1) (layer "B.Cu") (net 1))
 (segment (start 143.25 62.75) (end 142.75 62.25) (width 1.2) (layer "B.Cu") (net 1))
 (segment (start 169.75 96.75) (end 166.8675 96.75) (width 0.9) (layer "B.Cu") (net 1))
 (segment (start 143.25 64) (end 143.25 62.75) (width 1.2) (layer "B.Cu") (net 1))
 (segment (start 148.84 63.975) (end 148.84 63.84) (width 1) (layer "B.Cu") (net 1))
 (segment (start 161.25 97) (end 164 97) (width 1) (layer "B.Cu") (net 1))
 (segment (start 161.54 107.79) (end 161.75 108) (width 1) (layer "B.Cu") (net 1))
 (segment (start 146.32 72.12) (end 146.32 74.43) (width 0.8) (layer "B.Cu") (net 1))
 (segment (start 146.32 69.68) (end 146.32 72.12) (width 1) (layer "B.Cu") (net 1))
 (segment (start 161.75 108) (end 168.25 108) (width 1) (layer "B.Cu") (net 1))
 (segment (start 168.25 104.5) (end 171.75 101) (width 1) (layer "B.Cu") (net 1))
 (segment (start 147 68.75) (end 146.5 69.25) (width 1) (layer "B.Cu") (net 1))
 (segment (start 145 79.25) (end 145 77.5) (width 1.2) (layer "B.Cu") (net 1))
 (segment (start 170 99.25) (end 170 97) (width 0.9) (layer "B.Cu") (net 1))
 (segment (start 168.25 108) (end 168.25 104.5) (width 1) (layer "B.Cu") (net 1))
 (segment (start 164 97) (end 164.6175 96.3825) (width 1) (layer "B.Cu") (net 1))
 (segment (start 145 77.5) (end 145 75.75) (width 1.2) (layer "B.Cu") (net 1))
 (segment (start 176 77.5) (end 176.5 78) (width 1.2) (layer "B.Cu") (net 1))
 (segment (start 155 107.79) (end 161.54 107.79) (width 1) (layer "B.Cu") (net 1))
 (segment (start 178.5 101) (end 171.75 101) (width 1.1) (layer "B.Cu") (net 1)))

